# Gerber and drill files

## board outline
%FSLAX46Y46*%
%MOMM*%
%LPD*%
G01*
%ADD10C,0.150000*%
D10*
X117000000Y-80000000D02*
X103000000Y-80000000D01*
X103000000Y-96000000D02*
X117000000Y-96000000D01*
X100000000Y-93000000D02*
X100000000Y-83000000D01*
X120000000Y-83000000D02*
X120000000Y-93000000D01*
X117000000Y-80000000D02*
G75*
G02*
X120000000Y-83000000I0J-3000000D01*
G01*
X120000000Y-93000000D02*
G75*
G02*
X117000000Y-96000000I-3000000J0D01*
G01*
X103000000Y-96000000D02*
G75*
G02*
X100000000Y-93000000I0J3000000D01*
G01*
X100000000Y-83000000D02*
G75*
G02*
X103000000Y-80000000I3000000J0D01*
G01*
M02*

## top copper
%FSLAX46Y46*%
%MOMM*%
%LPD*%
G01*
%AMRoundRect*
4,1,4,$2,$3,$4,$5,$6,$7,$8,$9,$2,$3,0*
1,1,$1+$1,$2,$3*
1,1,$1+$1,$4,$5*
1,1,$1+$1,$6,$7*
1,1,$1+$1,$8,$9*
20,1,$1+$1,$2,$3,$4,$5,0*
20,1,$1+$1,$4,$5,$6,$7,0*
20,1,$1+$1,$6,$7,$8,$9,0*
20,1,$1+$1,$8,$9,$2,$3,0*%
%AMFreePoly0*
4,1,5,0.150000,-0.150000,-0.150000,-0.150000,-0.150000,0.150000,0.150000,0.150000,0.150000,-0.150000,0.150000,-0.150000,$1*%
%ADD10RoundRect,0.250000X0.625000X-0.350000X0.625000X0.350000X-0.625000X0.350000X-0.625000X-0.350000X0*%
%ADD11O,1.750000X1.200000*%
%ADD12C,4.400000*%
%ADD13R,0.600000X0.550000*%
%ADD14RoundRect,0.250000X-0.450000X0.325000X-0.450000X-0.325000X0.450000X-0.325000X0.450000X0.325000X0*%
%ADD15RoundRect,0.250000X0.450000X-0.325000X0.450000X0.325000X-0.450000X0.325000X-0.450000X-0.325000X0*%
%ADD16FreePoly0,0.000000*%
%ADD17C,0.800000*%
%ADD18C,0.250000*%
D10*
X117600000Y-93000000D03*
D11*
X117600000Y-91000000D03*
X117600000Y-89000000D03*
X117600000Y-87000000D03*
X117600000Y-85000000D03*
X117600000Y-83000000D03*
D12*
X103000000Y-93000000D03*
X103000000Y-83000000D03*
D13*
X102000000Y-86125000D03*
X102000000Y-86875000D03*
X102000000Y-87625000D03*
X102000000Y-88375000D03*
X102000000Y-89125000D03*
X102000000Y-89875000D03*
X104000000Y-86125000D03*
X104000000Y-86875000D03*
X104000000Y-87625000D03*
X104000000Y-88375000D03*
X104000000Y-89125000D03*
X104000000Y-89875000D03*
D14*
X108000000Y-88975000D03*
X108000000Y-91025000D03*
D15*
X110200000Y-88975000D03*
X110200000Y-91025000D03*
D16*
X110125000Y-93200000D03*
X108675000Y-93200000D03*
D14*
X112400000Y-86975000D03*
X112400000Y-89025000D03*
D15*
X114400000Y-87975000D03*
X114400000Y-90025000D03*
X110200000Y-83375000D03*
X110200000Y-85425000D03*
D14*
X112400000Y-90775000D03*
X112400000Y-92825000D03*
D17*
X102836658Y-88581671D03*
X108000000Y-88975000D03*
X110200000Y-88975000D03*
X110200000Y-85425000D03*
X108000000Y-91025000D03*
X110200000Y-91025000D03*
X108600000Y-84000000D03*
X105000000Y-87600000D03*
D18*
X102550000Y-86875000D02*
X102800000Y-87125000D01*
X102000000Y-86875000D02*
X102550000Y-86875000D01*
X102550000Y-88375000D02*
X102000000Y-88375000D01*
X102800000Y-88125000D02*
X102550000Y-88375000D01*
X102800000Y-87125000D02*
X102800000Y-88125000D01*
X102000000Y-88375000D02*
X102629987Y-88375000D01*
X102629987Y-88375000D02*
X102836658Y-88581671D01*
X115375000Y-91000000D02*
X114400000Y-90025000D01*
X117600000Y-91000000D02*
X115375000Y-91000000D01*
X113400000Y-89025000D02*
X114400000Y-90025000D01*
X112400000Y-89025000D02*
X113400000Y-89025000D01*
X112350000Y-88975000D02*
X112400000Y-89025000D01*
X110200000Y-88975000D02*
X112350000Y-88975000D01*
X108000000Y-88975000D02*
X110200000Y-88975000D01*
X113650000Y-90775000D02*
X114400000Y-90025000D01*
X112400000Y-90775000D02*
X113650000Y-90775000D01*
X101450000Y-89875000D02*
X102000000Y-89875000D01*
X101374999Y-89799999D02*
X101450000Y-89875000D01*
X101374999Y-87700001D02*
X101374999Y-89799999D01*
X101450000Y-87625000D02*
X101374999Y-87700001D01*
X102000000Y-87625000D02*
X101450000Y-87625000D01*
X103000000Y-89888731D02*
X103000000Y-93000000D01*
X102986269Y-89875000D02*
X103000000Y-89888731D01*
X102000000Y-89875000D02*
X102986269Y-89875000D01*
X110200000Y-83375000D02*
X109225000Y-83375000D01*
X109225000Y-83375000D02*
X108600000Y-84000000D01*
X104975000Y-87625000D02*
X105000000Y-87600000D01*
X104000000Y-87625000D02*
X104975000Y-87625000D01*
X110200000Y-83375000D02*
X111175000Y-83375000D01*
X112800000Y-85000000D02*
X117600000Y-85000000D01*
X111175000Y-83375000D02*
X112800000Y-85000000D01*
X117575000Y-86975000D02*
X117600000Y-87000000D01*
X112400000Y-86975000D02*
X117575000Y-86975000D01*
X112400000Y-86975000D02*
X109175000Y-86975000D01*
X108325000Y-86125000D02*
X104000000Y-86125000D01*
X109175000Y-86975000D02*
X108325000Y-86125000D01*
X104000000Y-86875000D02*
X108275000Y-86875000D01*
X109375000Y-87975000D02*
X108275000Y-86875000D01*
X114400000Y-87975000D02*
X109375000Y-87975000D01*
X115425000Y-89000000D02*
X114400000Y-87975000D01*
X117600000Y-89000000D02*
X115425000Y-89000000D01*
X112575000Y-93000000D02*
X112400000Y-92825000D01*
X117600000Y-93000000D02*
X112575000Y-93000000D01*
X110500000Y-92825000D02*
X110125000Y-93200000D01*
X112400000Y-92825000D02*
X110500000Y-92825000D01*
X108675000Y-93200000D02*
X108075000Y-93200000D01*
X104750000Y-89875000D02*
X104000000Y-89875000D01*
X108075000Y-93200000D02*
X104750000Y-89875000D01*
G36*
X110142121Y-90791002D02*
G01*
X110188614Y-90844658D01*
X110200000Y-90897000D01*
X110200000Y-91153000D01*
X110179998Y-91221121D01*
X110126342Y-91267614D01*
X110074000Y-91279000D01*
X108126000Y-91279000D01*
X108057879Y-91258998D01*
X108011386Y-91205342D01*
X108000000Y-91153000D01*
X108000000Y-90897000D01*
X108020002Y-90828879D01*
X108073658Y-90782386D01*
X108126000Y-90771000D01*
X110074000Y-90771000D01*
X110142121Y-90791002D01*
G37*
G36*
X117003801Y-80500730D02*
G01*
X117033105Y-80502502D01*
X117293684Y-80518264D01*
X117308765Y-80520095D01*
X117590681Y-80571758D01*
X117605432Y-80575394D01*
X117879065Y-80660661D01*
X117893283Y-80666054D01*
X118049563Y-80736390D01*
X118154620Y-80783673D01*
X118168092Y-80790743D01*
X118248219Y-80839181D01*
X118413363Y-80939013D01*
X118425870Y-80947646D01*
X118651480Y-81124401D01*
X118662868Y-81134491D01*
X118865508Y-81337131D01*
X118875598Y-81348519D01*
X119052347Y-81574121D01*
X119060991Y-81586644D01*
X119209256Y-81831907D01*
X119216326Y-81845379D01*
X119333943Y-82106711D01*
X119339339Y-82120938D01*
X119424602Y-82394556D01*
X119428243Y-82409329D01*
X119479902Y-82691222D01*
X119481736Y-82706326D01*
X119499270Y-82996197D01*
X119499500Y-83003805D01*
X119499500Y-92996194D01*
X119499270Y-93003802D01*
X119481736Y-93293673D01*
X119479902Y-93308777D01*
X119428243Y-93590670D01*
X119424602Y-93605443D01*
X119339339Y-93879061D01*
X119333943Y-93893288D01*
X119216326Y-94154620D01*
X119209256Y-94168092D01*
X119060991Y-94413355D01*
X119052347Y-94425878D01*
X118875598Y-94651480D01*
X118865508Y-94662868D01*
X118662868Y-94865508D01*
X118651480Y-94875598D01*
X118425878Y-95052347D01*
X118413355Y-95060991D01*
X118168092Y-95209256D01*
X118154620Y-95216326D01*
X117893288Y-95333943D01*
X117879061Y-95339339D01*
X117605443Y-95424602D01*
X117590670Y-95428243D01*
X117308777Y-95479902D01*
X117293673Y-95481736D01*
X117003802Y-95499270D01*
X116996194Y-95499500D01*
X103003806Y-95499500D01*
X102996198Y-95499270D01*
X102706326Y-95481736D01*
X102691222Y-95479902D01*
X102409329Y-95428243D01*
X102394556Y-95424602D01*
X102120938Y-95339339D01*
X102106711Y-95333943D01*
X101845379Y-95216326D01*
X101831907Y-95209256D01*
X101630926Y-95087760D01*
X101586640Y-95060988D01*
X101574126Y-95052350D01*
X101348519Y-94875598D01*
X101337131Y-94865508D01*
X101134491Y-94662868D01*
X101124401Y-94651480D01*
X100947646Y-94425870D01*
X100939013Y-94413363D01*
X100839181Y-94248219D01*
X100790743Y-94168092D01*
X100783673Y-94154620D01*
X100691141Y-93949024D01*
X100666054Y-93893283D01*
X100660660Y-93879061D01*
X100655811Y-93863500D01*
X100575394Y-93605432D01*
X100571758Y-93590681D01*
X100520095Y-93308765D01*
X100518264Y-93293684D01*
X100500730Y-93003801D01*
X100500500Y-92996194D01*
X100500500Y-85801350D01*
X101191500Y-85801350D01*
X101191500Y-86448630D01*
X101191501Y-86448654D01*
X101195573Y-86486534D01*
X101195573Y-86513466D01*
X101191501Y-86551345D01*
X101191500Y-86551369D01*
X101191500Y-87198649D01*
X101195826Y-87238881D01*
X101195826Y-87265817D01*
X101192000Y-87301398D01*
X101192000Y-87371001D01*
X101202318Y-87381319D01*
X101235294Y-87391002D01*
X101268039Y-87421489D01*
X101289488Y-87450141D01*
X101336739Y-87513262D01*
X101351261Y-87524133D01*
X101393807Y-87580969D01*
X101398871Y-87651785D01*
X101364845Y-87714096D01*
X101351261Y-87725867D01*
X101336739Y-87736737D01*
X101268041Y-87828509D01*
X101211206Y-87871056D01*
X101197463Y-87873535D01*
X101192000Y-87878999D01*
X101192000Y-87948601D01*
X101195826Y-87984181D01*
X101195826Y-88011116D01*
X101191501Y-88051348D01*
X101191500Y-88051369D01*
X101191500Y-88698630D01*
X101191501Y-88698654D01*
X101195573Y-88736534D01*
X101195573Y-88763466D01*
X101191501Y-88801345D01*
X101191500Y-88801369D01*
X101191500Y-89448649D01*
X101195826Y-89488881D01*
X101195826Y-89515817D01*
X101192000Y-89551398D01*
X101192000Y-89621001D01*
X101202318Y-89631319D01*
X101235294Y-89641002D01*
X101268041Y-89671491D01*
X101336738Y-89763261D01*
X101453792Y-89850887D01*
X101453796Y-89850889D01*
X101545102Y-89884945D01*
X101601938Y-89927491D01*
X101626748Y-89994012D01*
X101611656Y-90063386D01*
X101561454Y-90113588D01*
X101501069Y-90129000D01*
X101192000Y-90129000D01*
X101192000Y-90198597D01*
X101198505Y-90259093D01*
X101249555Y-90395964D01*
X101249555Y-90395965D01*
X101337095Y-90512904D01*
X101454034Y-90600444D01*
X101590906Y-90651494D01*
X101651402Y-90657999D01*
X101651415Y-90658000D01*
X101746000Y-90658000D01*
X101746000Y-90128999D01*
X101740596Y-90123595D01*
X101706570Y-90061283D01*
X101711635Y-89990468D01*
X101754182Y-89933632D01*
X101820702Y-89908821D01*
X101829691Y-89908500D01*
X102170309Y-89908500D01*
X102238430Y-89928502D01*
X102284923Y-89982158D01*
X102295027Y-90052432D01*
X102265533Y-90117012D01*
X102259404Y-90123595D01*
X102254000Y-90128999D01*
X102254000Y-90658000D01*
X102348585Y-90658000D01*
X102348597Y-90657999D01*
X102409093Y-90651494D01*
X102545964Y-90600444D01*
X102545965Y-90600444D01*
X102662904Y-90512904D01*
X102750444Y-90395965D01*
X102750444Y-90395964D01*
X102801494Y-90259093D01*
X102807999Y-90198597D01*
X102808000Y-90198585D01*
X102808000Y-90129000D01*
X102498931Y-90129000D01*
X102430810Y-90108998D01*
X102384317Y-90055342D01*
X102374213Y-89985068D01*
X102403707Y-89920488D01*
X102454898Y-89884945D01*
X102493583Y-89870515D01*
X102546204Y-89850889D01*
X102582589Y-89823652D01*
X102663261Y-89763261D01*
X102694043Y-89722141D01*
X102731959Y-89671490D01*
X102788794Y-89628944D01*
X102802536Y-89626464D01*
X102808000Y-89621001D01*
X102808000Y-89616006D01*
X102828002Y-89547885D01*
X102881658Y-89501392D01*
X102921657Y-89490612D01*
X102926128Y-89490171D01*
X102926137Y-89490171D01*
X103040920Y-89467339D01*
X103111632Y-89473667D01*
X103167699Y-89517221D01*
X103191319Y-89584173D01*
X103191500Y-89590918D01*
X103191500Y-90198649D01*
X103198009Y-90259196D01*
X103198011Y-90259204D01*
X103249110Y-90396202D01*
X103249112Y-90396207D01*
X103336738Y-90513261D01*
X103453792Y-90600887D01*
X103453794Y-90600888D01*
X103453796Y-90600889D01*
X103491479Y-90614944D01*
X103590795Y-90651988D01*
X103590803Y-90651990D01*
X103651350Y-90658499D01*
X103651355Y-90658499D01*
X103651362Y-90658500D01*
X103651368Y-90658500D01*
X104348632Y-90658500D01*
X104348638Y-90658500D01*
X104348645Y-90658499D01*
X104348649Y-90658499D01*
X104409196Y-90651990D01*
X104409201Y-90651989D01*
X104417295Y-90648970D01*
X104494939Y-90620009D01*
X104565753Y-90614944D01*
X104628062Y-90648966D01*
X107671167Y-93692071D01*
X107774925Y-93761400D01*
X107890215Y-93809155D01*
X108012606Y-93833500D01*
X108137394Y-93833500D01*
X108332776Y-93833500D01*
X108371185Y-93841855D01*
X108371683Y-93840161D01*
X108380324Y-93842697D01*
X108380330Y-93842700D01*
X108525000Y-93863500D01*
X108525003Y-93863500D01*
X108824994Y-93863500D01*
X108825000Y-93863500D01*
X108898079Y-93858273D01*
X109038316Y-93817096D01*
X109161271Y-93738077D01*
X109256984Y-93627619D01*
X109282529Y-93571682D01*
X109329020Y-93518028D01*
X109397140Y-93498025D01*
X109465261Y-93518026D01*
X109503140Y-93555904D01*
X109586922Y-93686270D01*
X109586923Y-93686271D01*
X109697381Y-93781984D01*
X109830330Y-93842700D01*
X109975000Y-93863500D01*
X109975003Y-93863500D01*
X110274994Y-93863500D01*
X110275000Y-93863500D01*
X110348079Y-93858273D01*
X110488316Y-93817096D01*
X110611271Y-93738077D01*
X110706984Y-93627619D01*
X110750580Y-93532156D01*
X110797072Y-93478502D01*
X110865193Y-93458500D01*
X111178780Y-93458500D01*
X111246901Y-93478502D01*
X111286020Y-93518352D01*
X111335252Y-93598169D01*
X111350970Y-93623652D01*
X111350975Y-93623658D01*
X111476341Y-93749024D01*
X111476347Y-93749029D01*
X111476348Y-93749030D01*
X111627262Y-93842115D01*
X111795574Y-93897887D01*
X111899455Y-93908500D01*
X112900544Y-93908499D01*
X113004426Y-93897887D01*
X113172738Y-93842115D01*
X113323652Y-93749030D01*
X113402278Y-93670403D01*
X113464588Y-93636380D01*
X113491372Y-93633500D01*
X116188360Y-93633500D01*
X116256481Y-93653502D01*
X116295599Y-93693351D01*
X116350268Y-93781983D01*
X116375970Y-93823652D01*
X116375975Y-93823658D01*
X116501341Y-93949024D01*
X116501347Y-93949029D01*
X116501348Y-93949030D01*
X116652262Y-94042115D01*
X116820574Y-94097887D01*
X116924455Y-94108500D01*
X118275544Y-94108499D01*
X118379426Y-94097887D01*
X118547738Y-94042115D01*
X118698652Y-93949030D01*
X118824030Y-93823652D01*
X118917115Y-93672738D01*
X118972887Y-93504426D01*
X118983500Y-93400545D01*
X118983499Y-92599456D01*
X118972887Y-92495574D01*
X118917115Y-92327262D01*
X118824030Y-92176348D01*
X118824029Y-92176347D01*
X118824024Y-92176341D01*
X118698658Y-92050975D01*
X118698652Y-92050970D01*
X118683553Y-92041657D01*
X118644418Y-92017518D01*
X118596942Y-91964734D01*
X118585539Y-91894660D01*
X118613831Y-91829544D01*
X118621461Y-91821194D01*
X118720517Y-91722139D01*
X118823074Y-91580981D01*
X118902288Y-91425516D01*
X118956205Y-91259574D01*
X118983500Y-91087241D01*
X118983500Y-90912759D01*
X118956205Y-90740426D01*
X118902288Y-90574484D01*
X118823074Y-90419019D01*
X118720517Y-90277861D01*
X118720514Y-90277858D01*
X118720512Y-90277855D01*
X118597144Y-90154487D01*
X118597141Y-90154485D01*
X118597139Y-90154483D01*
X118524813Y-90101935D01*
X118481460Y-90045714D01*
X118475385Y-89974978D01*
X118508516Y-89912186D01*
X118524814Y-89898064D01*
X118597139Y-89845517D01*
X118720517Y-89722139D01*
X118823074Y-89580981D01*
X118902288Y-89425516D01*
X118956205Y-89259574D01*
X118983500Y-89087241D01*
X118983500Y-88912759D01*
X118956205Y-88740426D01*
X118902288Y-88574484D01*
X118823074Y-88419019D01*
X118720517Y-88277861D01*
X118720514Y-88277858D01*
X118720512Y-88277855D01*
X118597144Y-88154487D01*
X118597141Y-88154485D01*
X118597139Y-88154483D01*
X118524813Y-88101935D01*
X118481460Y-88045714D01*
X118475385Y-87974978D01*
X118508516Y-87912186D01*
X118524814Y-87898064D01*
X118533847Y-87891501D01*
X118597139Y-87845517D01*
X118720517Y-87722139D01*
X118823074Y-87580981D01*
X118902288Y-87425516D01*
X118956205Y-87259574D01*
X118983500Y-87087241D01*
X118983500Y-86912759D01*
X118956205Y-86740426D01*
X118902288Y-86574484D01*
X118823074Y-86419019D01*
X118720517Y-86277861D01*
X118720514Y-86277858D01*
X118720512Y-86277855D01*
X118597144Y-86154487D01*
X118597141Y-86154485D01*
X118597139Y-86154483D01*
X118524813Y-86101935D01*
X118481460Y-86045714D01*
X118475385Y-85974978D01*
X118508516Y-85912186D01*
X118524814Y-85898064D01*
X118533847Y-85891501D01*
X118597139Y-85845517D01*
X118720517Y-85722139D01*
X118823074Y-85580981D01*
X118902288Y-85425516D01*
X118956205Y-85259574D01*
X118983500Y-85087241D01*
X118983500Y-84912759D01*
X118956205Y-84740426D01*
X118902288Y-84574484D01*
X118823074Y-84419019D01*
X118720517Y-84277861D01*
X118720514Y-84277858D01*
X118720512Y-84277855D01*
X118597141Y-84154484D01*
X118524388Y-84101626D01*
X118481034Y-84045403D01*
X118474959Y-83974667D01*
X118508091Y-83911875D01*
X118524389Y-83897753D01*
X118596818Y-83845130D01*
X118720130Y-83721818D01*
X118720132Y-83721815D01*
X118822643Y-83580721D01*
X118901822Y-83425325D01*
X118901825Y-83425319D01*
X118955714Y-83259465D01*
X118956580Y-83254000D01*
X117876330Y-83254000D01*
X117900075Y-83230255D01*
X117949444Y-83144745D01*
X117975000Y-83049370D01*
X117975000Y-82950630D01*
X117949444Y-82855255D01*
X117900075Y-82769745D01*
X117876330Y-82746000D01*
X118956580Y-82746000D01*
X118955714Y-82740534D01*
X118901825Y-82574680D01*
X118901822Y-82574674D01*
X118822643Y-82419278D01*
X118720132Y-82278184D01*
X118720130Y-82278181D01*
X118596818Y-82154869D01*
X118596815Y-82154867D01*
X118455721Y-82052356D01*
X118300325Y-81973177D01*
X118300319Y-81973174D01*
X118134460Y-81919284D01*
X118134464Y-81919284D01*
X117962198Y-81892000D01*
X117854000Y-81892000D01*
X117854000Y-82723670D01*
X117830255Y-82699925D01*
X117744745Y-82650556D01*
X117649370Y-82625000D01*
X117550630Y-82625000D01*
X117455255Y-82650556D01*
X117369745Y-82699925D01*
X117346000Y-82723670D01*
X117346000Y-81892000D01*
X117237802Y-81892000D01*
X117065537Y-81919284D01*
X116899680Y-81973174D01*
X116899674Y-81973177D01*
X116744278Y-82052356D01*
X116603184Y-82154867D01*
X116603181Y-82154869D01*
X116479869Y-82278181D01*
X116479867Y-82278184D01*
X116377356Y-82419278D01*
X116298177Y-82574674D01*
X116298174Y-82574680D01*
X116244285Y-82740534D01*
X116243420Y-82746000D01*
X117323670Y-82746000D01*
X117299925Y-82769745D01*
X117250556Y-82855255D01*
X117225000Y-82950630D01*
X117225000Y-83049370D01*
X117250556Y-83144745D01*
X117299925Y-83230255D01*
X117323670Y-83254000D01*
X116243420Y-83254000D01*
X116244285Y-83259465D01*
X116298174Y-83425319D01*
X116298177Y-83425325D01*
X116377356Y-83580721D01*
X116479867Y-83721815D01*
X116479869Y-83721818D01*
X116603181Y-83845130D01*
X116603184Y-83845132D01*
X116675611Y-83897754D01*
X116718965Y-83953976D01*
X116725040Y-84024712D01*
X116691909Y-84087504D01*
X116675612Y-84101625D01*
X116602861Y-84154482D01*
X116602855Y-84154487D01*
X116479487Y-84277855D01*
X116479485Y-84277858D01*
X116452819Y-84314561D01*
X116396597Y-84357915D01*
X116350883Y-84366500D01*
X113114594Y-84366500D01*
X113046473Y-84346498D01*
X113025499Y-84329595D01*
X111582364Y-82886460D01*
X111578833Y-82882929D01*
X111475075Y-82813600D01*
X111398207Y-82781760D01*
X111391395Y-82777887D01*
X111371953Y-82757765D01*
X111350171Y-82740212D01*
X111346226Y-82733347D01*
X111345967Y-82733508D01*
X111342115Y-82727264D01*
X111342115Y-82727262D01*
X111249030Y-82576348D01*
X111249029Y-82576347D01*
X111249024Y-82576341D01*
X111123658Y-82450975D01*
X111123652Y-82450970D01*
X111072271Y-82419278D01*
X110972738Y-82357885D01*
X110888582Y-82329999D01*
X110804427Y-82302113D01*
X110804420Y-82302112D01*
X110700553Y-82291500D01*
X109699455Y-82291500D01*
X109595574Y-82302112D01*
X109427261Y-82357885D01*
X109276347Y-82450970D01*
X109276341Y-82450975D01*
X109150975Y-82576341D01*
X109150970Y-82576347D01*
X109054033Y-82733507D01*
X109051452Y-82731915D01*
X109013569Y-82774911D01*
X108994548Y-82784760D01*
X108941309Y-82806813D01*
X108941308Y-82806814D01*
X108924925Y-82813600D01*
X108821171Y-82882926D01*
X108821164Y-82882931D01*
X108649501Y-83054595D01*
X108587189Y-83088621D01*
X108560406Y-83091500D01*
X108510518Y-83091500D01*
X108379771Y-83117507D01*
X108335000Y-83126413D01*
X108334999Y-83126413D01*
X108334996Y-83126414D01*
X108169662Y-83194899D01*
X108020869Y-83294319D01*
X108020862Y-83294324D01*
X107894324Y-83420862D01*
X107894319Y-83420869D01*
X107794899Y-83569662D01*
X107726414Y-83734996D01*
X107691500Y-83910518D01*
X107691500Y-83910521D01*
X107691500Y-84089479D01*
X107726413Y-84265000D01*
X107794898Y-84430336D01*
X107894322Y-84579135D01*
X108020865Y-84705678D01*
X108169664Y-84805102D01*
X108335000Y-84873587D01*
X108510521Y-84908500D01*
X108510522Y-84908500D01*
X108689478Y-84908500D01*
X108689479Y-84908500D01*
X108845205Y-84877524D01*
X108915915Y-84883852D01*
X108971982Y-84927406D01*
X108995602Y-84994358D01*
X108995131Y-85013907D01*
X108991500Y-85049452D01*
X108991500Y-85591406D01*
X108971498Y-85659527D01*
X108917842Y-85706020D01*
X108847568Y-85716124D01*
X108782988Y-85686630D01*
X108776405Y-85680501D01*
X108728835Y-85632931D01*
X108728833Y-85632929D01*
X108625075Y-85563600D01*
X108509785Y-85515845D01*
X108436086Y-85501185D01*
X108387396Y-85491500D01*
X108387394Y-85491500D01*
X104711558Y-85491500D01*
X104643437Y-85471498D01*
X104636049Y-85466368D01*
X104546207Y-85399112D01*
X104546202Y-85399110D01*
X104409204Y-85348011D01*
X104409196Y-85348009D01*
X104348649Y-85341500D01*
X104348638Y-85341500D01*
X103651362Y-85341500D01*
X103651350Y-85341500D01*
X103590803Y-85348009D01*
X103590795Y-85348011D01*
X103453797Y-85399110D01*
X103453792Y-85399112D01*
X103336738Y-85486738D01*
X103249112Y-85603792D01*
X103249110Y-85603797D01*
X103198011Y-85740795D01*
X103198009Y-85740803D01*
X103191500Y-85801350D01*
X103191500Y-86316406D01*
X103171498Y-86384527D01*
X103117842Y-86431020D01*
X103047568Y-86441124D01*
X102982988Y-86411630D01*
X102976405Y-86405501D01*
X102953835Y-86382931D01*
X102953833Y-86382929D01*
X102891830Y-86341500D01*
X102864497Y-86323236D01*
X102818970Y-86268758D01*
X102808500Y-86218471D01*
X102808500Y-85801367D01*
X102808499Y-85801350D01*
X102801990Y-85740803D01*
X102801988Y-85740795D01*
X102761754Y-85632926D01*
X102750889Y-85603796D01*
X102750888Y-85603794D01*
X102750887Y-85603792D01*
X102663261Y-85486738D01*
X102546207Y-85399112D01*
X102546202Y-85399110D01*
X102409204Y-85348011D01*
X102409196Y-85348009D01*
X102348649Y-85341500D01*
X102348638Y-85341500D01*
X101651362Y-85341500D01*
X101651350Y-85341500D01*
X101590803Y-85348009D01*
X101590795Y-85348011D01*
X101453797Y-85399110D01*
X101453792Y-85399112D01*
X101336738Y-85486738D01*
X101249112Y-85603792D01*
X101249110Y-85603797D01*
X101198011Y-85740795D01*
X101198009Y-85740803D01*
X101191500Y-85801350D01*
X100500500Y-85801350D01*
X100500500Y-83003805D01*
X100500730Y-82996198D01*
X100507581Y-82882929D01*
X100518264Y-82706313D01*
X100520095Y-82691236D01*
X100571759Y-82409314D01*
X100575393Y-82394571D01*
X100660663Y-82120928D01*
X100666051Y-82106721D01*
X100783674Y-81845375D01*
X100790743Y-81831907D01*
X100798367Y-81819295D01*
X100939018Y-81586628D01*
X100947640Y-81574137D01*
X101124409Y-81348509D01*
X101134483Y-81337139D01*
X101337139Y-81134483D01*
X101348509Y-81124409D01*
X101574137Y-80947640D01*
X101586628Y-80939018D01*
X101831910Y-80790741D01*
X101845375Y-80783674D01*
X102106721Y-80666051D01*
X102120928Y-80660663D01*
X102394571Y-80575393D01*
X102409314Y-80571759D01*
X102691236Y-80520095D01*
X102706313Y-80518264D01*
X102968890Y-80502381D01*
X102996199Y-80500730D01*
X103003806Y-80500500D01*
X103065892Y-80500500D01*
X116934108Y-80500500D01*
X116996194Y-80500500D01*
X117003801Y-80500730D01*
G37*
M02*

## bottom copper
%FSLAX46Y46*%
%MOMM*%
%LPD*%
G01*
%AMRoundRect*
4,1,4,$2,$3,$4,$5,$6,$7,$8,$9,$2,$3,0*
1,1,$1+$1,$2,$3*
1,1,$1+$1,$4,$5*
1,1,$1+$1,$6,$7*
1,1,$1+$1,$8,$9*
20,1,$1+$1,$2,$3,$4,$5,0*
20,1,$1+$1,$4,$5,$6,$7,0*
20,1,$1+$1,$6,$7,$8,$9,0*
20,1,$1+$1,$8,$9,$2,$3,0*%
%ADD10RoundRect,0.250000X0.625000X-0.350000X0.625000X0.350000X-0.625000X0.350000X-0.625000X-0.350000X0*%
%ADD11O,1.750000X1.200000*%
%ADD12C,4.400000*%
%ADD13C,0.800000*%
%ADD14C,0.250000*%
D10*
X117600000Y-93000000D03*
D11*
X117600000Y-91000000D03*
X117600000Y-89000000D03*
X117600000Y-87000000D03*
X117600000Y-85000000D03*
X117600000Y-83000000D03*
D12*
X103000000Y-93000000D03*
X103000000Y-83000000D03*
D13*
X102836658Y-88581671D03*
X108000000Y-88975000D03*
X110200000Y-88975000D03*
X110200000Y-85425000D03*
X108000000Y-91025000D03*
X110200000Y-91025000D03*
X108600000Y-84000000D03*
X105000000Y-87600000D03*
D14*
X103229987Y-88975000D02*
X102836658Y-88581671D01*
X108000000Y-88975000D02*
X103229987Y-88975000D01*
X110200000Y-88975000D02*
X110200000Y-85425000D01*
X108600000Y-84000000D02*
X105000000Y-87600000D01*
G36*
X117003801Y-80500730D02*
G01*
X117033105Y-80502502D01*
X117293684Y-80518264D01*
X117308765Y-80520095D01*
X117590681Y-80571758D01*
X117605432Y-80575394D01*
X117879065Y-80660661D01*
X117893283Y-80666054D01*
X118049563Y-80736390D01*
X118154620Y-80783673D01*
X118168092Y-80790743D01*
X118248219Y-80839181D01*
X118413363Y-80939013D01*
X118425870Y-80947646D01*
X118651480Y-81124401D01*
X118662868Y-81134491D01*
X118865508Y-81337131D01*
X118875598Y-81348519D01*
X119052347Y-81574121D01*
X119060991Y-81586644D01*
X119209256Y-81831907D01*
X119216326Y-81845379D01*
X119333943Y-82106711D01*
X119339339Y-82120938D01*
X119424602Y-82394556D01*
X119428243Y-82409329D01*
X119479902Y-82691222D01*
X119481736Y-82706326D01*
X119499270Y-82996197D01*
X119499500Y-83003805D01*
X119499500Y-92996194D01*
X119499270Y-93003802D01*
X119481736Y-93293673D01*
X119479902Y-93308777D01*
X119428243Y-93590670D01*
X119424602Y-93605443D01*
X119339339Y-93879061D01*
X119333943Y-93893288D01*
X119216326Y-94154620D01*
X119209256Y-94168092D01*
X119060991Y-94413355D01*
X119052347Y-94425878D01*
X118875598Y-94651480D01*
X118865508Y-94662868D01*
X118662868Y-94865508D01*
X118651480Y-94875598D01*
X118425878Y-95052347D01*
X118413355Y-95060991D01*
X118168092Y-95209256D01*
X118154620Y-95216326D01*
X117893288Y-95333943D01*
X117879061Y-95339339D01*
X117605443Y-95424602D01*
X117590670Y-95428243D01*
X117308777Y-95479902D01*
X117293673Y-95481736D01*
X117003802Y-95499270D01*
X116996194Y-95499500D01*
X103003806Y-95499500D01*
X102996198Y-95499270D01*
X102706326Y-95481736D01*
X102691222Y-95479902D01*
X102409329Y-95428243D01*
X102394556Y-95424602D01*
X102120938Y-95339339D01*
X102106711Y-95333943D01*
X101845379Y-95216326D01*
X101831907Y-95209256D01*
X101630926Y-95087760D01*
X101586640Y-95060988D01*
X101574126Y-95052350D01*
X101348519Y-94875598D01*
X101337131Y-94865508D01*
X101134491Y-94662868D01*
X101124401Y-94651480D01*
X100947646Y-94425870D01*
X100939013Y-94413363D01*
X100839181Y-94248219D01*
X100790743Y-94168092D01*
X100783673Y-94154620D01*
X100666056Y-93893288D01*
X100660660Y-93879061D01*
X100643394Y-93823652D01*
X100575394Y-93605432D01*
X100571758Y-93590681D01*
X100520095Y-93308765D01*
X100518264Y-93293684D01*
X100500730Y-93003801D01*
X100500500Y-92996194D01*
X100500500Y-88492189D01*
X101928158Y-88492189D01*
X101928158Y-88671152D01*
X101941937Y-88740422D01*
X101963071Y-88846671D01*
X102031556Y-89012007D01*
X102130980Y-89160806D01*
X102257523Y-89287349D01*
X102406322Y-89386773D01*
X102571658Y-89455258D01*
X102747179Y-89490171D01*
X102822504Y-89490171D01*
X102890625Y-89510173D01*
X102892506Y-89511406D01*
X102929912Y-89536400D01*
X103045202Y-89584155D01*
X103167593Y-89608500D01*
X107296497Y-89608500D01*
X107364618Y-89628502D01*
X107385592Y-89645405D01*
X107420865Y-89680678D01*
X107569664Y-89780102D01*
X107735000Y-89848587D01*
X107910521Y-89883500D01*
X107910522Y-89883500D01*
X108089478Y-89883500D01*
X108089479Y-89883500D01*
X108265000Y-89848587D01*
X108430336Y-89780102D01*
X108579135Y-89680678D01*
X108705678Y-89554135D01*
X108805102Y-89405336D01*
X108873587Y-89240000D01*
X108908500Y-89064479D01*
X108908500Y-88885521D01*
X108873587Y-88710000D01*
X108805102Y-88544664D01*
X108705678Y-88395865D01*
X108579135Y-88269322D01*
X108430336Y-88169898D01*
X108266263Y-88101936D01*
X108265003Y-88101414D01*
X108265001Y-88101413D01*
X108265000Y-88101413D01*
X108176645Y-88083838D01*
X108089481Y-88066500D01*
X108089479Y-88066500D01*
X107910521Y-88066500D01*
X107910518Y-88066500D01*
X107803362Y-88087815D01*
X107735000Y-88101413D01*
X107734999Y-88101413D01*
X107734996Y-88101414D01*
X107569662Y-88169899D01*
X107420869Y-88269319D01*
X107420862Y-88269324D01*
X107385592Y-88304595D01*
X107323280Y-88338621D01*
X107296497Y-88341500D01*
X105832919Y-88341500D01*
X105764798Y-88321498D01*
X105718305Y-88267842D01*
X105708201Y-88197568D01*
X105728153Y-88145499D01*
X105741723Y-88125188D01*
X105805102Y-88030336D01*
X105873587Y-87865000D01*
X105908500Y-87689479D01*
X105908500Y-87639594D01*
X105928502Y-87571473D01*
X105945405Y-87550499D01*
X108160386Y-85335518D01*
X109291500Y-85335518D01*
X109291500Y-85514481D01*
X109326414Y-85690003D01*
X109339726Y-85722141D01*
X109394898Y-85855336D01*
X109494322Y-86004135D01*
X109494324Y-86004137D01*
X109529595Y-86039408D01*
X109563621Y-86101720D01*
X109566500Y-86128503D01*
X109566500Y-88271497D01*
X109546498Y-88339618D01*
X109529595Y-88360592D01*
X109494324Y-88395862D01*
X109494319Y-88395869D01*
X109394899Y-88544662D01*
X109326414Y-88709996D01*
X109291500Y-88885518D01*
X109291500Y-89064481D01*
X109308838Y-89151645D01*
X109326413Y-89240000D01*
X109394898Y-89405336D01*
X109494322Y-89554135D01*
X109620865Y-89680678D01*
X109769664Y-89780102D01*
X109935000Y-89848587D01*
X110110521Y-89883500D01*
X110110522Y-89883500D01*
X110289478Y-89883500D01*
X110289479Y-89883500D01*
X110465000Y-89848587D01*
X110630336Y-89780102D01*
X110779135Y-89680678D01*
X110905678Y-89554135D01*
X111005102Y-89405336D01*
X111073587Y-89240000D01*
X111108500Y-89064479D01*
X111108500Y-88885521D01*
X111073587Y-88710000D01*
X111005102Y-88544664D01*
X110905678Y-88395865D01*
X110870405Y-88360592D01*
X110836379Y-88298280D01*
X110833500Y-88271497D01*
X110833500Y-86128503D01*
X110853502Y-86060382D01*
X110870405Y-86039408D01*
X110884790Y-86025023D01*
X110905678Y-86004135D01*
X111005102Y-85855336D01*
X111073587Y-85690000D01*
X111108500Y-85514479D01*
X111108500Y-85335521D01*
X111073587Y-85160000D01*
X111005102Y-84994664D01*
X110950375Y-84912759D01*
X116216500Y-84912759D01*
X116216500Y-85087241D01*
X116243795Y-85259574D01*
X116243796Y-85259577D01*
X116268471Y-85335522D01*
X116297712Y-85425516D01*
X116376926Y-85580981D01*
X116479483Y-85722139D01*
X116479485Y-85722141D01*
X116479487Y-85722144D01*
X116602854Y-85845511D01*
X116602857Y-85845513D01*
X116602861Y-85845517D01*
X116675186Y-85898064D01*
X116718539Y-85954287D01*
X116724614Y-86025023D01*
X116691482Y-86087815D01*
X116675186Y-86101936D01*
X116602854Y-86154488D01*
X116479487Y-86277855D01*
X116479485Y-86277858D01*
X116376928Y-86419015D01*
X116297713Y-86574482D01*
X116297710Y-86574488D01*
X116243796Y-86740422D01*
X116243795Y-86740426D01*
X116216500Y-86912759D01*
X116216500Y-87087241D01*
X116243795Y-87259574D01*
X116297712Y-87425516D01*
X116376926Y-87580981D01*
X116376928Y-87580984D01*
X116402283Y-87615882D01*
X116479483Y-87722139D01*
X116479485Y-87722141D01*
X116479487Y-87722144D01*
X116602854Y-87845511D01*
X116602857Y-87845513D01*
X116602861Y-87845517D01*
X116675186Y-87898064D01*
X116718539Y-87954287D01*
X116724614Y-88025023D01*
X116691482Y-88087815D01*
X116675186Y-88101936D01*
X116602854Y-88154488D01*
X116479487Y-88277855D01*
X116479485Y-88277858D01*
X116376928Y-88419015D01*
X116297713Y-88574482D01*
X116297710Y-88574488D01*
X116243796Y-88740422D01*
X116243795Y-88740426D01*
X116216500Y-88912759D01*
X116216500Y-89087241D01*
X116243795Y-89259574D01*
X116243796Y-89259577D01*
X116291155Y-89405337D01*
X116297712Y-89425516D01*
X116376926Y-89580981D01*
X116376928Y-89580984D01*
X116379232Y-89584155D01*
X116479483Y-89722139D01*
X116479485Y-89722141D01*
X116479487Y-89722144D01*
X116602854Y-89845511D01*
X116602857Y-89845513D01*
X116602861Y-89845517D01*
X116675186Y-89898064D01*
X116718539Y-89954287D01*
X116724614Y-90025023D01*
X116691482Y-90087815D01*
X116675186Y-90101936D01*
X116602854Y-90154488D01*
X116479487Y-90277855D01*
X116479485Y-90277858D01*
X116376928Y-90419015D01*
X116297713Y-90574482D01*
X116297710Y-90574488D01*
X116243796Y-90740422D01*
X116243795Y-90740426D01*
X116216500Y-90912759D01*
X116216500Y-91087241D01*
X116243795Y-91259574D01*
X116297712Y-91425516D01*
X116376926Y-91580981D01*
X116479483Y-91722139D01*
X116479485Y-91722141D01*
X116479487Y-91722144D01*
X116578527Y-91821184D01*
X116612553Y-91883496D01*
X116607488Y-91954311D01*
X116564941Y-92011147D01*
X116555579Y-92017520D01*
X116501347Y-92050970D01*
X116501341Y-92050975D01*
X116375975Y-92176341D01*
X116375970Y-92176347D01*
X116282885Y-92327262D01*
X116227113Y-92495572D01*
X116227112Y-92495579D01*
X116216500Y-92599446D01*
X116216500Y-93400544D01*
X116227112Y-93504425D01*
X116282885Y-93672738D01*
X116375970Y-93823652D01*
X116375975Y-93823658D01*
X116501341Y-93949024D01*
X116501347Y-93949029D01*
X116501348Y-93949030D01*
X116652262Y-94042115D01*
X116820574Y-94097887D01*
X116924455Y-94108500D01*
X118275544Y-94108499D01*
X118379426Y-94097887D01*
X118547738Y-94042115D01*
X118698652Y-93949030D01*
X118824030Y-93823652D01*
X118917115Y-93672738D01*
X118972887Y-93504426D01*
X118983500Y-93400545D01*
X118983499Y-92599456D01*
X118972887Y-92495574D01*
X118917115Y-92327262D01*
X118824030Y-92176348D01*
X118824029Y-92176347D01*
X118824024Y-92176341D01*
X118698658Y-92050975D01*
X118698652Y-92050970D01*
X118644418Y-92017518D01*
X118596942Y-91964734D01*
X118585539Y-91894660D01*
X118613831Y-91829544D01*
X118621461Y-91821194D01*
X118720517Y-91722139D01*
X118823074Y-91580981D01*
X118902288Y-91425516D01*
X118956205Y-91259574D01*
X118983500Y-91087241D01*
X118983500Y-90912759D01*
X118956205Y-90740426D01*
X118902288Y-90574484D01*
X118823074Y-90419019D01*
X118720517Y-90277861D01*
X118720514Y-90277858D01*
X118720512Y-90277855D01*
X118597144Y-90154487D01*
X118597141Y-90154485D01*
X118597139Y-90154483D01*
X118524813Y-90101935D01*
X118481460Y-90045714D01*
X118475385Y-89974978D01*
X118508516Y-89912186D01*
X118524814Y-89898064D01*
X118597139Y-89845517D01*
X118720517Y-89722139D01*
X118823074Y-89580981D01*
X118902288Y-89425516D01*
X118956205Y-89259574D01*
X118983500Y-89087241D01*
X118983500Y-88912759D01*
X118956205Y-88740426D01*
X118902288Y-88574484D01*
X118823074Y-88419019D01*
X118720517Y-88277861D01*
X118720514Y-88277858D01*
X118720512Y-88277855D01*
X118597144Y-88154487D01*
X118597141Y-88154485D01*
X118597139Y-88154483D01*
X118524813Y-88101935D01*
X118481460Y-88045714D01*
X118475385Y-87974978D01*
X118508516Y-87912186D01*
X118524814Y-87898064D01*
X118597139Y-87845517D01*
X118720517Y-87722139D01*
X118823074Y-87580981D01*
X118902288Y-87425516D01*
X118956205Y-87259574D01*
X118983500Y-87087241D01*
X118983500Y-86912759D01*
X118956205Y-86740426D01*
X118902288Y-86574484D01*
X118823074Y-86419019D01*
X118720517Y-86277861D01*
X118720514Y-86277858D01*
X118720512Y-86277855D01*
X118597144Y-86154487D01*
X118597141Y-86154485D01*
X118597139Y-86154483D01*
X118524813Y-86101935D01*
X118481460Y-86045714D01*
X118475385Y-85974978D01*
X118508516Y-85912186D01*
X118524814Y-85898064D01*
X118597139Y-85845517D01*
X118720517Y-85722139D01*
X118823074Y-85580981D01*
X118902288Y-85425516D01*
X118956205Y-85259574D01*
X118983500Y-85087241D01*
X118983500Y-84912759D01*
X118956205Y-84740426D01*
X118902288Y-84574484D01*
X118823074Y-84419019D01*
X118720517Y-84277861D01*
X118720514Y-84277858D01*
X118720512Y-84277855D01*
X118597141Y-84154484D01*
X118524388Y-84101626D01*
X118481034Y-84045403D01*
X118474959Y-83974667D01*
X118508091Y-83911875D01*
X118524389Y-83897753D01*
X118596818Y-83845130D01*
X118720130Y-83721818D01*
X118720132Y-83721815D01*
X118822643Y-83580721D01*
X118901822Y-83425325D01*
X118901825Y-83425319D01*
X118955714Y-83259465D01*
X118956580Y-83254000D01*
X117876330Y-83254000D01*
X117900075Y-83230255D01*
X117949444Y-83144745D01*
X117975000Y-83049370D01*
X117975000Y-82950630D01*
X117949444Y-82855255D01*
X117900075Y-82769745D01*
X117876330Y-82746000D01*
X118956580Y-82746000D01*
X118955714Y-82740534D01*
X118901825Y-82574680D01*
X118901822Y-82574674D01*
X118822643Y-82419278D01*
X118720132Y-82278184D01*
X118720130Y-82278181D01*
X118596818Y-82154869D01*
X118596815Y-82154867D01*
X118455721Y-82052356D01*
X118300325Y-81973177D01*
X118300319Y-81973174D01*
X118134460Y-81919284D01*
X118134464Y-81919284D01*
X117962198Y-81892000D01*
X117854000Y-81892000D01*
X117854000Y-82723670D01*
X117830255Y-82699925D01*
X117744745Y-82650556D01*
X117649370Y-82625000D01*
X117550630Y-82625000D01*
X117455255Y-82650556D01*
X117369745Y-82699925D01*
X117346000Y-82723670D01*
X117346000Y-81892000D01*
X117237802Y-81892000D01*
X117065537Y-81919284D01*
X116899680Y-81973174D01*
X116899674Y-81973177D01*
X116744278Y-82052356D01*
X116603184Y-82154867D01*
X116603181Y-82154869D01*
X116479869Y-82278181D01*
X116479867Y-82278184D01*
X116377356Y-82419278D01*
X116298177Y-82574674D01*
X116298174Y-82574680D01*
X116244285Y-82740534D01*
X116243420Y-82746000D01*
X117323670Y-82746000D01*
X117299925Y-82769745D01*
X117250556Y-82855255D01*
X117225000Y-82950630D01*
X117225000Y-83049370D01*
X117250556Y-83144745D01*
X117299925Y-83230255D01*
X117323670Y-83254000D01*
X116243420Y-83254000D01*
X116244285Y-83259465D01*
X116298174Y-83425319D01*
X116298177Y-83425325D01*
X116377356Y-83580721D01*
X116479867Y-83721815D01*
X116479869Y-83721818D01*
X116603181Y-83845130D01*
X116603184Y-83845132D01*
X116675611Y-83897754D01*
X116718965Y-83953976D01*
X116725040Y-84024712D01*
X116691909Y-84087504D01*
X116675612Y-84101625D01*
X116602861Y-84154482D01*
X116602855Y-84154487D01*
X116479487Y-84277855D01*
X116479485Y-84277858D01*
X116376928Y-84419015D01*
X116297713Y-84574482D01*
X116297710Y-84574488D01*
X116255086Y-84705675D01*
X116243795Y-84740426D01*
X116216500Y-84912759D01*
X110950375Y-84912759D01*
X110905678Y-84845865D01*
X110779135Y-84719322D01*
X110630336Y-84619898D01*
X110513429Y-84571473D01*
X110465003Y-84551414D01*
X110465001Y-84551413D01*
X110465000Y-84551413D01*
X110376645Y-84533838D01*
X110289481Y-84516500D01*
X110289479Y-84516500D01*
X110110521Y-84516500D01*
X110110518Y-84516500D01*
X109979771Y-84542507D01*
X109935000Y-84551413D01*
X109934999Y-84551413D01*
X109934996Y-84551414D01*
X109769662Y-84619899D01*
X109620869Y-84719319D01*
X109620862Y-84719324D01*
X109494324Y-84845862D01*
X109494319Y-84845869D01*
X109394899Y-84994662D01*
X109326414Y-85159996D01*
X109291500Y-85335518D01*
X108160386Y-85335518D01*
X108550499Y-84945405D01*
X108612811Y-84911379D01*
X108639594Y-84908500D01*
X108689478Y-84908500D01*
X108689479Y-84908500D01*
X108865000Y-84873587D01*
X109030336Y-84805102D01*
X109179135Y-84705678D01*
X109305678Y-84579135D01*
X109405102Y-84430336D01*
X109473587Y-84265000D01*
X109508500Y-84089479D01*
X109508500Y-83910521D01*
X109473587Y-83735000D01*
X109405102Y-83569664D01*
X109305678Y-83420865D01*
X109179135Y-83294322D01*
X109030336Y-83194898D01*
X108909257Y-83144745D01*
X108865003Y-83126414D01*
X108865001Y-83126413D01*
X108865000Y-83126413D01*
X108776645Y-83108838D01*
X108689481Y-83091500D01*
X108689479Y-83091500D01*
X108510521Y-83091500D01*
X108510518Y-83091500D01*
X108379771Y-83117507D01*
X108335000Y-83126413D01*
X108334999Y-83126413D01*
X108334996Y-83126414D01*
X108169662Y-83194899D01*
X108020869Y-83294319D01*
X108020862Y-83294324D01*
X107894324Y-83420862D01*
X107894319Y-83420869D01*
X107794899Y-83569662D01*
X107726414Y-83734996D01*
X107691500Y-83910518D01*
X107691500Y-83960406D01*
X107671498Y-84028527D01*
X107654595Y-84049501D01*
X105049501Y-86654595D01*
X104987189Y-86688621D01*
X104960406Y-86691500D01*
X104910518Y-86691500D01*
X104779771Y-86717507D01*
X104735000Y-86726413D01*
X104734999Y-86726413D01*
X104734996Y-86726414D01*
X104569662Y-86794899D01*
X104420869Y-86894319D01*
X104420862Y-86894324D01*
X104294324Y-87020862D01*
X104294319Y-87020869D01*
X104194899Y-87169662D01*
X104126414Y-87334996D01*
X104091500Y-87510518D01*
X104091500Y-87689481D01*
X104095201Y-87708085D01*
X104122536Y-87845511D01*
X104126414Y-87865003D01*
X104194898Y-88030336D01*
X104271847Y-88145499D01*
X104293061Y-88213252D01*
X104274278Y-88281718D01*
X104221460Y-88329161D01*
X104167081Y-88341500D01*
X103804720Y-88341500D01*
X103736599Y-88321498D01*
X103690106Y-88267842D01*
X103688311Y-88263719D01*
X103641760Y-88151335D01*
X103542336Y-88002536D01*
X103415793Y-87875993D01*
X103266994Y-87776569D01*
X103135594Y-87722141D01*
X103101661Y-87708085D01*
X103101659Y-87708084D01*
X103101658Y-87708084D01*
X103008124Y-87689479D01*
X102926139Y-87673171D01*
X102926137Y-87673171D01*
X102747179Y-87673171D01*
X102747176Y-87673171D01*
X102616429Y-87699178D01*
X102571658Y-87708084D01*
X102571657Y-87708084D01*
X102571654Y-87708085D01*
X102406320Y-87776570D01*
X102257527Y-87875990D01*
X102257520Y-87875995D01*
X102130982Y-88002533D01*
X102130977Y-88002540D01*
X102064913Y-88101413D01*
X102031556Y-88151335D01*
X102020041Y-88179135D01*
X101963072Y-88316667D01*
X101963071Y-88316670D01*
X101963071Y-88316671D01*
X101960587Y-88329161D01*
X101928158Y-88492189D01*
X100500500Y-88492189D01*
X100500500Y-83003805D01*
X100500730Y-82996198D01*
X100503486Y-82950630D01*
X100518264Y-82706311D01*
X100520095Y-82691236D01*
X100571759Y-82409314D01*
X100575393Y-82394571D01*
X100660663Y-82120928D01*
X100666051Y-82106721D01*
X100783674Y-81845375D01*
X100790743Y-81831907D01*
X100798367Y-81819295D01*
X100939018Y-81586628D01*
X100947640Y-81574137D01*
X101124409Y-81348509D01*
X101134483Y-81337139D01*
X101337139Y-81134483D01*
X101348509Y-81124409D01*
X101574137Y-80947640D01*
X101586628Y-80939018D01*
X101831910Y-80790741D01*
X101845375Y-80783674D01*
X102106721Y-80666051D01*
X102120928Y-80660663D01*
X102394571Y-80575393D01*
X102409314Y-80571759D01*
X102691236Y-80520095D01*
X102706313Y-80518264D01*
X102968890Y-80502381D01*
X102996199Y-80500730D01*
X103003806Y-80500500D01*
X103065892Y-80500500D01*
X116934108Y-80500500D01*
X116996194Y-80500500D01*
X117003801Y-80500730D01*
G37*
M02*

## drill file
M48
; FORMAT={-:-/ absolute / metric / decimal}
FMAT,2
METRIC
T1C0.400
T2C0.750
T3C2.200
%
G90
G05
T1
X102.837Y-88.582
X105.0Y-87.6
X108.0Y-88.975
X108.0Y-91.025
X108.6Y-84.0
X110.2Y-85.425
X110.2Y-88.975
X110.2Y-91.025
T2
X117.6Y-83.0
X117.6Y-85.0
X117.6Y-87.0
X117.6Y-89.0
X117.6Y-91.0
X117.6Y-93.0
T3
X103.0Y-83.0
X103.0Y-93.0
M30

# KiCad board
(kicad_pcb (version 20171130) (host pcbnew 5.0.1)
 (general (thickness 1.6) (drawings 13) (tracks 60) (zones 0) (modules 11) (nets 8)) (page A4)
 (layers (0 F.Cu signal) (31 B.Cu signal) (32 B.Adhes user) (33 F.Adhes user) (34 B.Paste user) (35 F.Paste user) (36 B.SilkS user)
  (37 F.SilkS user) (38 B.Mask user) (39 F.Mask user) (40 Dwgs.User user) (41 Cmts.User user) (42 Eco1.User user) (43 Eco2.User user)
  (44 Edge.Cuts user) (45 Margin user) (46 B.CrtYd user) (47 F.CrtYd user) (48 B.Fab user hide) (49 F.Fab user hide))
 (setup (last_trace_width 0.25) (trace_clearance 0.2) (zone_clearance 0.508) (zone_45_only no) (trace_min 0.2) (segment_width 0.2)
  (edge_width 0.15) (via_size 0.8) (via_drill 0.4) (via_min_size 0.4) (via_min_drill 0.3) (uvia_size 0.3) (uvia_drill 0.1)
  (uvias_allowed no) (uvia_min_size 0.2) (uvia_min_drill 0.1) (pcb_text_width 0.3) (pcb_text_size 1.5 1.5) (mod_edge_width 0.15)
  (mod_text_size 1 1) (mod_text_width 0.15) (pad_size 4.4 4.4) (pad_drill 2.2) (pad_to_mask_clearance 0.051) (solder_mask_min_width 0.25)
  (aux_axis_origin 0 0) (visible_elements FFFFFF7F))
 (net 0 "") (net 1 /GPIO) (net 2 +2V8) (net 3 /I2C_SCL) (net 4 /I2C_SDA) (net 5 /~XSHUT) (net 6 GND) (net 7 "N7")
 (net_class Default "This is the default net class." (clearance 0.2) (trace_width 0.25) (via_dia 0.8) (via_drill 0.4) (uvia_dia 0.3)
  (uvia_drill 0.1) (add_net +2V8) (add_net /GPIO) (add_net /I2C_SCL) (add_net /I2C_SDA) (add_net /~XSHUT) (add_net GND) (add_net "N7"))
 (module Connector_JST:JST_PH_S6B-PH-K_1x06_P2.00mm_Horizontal (layer B.Cu) (at 117.6 93 90)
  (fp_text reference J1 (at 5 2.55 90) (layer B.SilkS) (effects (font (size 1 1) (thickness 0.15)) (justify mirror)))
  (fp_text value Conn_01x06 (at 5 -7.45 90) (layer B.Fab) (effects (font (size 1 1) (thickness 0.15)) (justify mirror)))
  (pad 1 thru_hole roundrect (at 0 0 90) (size 1.2 1.75) (drill 0.75) (layers *.Cu *.Mask) (roundrect_rratio 0.208333) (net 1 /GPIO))
  (pad 2 thru_hole oval (at 2 0 90) (size 1.2 1.75) (drill 0.75) (layers *.Cu *.Mask) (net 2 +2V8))
  (pad 3 thru_hole oval (at 4 0 90) (size 1.2 1.75) (drill 0.75) (layers *.Cu *.Mask) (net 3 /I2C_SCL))
  (pad 4 thru_hole oval (at 6 0 90) (size 1.2 1.75) (drill 0.75) (layers *.Cu *.Mask) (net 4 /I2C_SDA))
  (pad 5 thru_hole oval (at 8 0 90) (size 1.2 1.75) (drill 0.75) (layers *.Cu *.Mask) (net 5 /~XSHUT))
  (pad 6 thru_hole oval (at 10 0 90) (size 1.2 1.75) (drill 0.75) (layers *.Cu *.Mask) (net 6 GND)))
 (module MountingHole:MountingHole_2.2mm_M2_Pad (layer F.Cu) (at 103 93)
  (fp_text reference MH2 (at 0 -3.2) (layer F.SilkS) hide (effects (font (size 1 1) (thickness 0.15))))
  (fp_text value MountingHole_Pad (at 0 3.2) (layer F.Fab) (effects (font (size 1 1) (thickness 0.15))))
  (pad 1 thru_hole circle (at 0 0) (size 4.4 4.4) (drill 2.2) (layers *.Cu *.Mask) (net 6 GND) (zone_connect 2)))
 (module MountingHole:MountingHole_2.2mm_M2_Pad (layer F.Cu) (at 103 83)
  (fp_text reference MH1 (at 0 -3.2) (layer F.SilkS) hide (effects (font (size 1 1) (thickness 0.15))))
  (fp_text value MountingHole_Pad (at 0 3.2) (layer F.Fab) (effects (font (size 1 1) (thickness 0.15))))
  (pad 1 thru_hole circle (at 0 0) (size 4.4 4.4) (drill 2.2) (layers *.Cu *.Mask) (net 6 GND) (zone_connect 2)))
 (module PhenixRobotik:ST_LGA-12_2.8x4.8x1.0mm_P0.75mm (layer F.Cu) (at 103 88 180)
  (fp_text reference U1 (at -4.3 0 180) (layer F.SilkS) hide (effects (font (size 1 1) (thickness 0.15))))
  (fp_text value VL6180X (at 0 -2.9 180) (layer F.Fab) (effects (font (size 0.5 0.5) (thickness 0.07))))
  (pad 7 smd rect (at 1 1.875) (size 0.6 0.55) (layers F.Cu F.Paste F.Mask))
  (pad 8 smd rect (at 1 1.125) (size 0.6 0.55) (layers F.Cu F.Paste F.Mask) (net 2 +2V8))
  (pad 9 smd rect (at 1 0.375) (size 0.6 0.55) (layers F.Cu F.Paste F.Mask) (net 6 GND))
  (pad 10 smd rect (at 1 -0.375) (size 0.6 0.55) (layers F.Cu F.Paste F.Mask) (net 2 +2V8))
  (pad 11 smd rect (at 1 -1.125) (size 0.6 0.55) (layers F.Cu F.Paste F.Mask))
  (pad 12 smd rect (at 1 -1.875) (size 0.6 0.55) (layers F.Cu F.Paste F.Mask) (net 6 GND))
  (pad 6 smd rect (at -1 1.875) (size 0.6 0.55) (layers F.Cu F.Paste F.Mask) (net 4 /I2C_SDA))
  (pad 5 smd rect (at -1 1.125) (size 0.6 0.55) (layers F.Cu F.Paste F.Mask) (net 3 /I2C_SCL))
  (pad 4 smd rect (at -1 0.375) (size 0.6 0.55) (layers F.Cu F.Paste F.Mask) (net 5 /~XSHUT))
  (pad 3 smd rect (at -1 -0.375) (size 0.6 0.55) (layers F.Cu F.Paste F.Mask))
  (pad 2 smd rect (at -1 -1.125) (size 0.6 0.55) (layers F.Cu F.Paste F.Mask))
  (pad 1 smd rect (at -1 -1.875) (size 0.6 0.55) (layers F.Cu F.Paste F.Mask) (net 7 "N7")))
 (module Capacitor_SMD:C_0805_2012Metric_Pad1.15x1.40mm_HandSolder (layer F.Cu) (at 108 90 270)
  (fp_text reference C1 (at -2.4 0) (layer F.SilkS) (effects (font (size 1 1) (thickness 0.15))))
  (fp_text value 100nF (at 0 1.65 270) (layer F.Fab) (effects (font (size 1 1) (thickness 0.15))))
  (pad 1 smd roundrect (at -1.025 0 270) (size 1.15 1.4) (layers F.Cu F.Paste F.Mask) (roundrect_rratio 0.217391) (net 2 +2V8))
  (pad 2 smd roundrect (at 1.025 0 270) (size 1.15 1.4) (layers F.Cu F.Paste F.Mask) (roundrect_rratio 0.217391) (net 6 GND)))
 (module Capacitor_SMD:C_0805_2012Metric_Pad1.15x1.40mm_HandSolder (layer F.Cu) (at 110.2 90 90)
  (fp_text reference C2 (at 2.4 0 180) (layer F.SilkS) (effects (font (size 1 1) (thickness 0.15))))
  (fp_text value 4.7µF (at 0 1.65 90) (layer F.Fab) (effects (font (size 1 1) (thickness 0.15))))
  (pad 2 smd roundrect (at 1.025 0 90) (size 1.15 1.4) (layers F.Cu F.Paste F.Mask) (roundrect_rratio 0.217391) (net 2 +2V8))
  (pad 1 smd roundrect (at -1.025 0 90) (size 1.15 1.4) (layers F.Cu F.Paste F.Mask) (roundrect_rratio 0.217391) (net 6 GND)))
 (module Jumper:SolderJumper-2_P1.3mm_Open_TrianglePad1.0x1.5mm (layer F.Cu) (at 109.4 93.2)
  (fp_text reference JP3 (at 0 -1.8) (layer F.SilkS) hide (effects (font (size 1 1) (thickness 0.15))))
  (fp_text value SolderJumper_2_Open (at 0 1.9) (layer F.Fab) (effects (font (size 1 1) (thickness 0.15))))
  (pad 2 smd custom (at 0.725 0) (size 0.3 0.3) (layers F.Cu F.Mask) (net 1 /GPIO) (zone_connect 0)
   (options (clearance outline) (anchor rect)) (primitives))
  (pad 1 smd custom (at -0.725 0) (size 0.3 0.3) (layers F.Cu F.Mask) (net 7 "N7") (zone_connect 0)
   (options (clearance outline) (anchor rect)) (primitives)))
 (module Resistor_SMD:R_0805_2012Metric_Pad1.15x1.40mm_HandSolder (layer F.Cu) (at 112.4 88 270)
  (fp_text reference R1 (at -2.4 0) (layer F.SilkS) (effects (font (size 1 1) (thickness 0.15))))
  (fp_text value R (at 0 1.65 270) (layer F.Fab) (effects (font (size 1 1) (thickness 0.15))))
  (pad 1 smd roundrect (at -1.025 0 270) (size 1.15 1.4) (layers F.Cu F.Paste F.Mask) (roundrect_rratio 0.217391) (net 4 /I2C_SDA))
  (pad 2 smd roundrect (at 1.025 0 270) (size 1.15 1.4) (layers F.Cu F.Paste F.Mask) (roundrect_rratio 0.217391) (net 2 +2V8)))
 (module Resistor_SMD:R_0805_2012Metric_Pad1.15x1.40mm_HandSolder (layer F.Cu) (at 114.4 89 90)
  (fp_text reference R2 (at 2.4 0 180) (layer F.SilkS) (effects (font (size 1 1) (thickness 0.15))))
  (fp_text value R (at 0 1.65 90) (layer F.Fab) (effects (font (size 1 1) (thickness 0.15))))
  (pad 2 smd roundrect (at 1.025 0 90) (size 1.15 1.4) (layers F.Cu F.Paste F.Mask) (roundrect_rratio 0.217391) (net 3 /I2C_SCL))
  (pad 1 smd roundrect (at -1.025 0 90) (size 1.15 1.4) (layers F.Cu F.Paste F.Mask) (roundrect_rratio 0.217391) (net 2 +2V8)))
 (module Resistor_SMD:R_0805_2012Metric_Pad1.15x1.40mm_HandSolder (layer F.Cu) (at 110.2 84.4 90)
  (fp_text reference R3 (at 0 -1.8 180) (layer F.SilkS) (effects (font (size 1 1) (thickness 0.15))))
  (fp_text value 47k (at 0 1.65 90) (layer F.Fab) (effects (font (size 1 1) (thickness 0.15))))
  (pad 2 smd roundrect (at 1.025 0 90) (size 1.15 1.4) (layers F.Cu F.Paste F.Mask) (roundrect_rratio 0.217391) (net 5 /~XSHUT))
  (pad 1 smd roundrect (at -1.025 0 90) (size 1.15 1.4) (layers F.Cu F.Paste F.Mask) (roundrect_rratio 0.217391) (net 2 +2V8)))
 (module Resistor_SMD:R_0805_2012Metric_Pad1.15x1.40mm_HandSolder (layer F.Cu) (at 112.4 91.8 270)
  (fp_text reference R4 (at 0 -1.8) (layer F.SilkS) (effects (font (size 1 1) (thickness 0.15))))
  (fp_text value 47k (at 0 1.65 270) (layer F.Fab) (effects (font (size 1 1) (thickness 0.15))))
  (pad 1 smd roundrect (at -1.025 0 270) (size 1.15 1.4) (layers F.Cu F.Paste F.Mask) (roundrect_rratio 0.217391) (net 2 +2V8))
  (pad 2 smd roundrect (at 1.025 0 270) (size 1.15 1.4) (layers F.Cu F.Paste F.Mask) (roundrect_rratio 0.217391) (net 1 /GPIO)))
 (gr_line (start 117 80) (end 103 80) (layer Edge.Cuts) (width 0.15))
 (gr_line (start 103 96) (end 117 96) (layer Edge.Cuts) (width 0.15))
 (gr_line (start 100 93) (end 100 83) (angle 90) (layer Edge.Cuts) (width 0.15))
 (gr_line (start 120 83) (end 120 93) (angle 90) (layer Edge.Cuts) (width 0.15))
 (gr_arc (start 117 83) (end 117 80) (angle 90) (layer Edge.Cuts) (width 0.15))
 (gr_arc (start 117 93) (end 120 93) (angle 90) (layer Edge.Cuts) (width 0.15))
 (gr_arc (start 103 93) (end 103 96) (angle 90) (layer Edge.Cuts) (width 0.15))
 (gr_arc (start 103 83) (end 100 83) (angle 90) (layer Edge.Cuts) (width 0.15))
 (segment (start 102.55 86.875) (end 102.8 87.125) (width 0.25) (layer F.Cu) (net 2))
 (segment (start 102 86.875) (end 102.55 86.875) (width 0.25) (layer F.Cu) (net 2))
 (segment (start 102.55 88.375) (end 102 88.375) (width 0.25) (layer F.Cu) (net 2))
 (segment (start 102.8 88.125) (end 102.55 88.375) (width 0.25) (layer F.Cu) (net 2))
 (segment (start 102.8 87.125) (end 102.8 88.125) (width 0.25) (layer F.Cu) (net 2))
 (via (at 102.836658 88.581671) (size 0.8) (drill 0.4) (layers F.Cu B.Cu) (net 2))
 (segment (start 102 88.375) (end 102.629987 88.375) (width 0.25) (layer F.Cu) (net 2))
 (segment (start 102.629987 88.375) (end 102.836658 88.581671) (width 0.25) (layer F.Cu) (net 2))
 (segment (start 115.375 91) (end 114.4 90.025) (width 0.25) (layer F.Cu) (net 2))
 (segment (start 117.6 91) (end 115.375 91) (width 0.25) (layer F.Cu) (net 2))
 (segment (start 113.4 89.025) (end 114.4 90.025) (width 0.25) (layer F.Cu) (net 2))
 (segment (start 112.4 89.025) (end 113.4 89.025) (width 0.25) (layer F.Cu) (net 2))
 (segment (start 112.35 88.975) (end 112.4 89.025) (width 0.25) (layer F.Cu) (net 2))
 (segment (start 110.2 88.975) (end 112.35 88.975) (width 0.25) (layer F.Cu) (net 2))
 (segment (start 108 88.975) (end 110.2 88.975) (width 0.25) (layer F.Cu) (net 2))
 (via (at 108 88.975) (size 0.8) (drill 0.4) (layers F.Cu B.Cu) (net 2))
 (segment (start 113.65 90.775) (end 114.4 90.025) (width 0.25) (layer F.Cu) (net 2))
 (segment (start 112.4 90.775) (end 113.65 90.775) (width 0.25) (layer F.Cu) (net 2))
 (segment (start 103.229987 88.975) (end 102.836658 88.581671) (width 0.25) (layer B.Cu) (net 2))
 (segment (start 108 88.975) (end 103.229987 88.975) (width 0.25) (layer B.Cu) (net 2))
 (via (at 110.2 88.975) (size 0.8) (drill 0.4) (layers F.Cu B.Cu) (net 2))
 (via (at 110.2 85.425) (size 0.8) (drill 0.4) (layers F.Cu B.Cu) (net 2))
 (segment (start 110.2 88.975) (end 110.2 85.425) (width 0.25) (layer B.Cu) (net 2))
 (segment (start 101.45 89.875) (end 102 89.875) (width 0.25) (layer F.Cu) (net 6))
 (segment (start 101.374999 89.799999) (end 101.45 89.875) (width 0.25) (layer F.Cu) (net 6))
 (segment (start 101.374999 87.700001) (end 101.374999 89.799999) (width 0.25) (layer F.Cu) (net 6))
 (segment (start 101.45 87.625) (end 101.374999 87.700001) (width 0.25) (layer F.Cu) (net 6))
 (segment (start 102 87.625) (end 101.45 87.625) (width 0.25) (layer F.Cu) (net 6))
 (segment (start 103 89.888731) (end 103 93) (width 0.25) (layer F.Cu) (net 6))
 (segment (start 102.986269 89.875) (end 103 89.888731) (width 0.25) (layer F.Cu) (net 6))
 (segment (start 102 89.875) (end 102.986269 89.875) (width 0.25) (layer F.Cu) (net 6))
 (via (at 108 91.025) (size 0.8) (drill 0.4) (layers F.Cu B.Cu) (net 6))
 (via (at 110.2 91.025) (size 0.8) (drill 0.4) (layers F.Cu B.Cu) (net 6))
 (via (at 108.6 84) (size 0.8) (drill 0.4) (layers F.Cu B.Cu) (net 5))
 (segment (start 110.2 83.375) (end 109.225 83.375) (width 0.25) (layer F.Cu) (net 5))
 (segment (start 109.225 83.375) (end 108.6 84) (width 0.25) (layer F.Cu) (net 5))
 (via (at 105 87.6) (size 0.8) (drill 0.4) (layers F.Cu B.Cu) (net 5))
 (segment (start 108.6 84) (end 105 87.6) (width 0.25) (layer B.Cu) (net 5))
 (segment (start 104.975 87.625) (end 105 87.6) (width 0.25) (layer F.Cu) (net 5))
 (segment (start 104 87.625) (end 104.975 87.625) (width 0.25) (layer F.Cu) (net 5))
 (segment (start 110.2 83.375) (end 111.175 83.375) (width 0.25) (layer F.Cu) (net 5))
 (segment (start 112.8 85) (end 117.6 85) (width 0.25) (layer F.Cu) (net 5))
 (segment (start 111.175 83.375) (end 112.8 85) (width 0.25) (layer F.Cu) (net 5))
 (segment (start 117.575 86.975) (end 117.6 87) (width 0.25) (layer F.Cu) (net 4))
 (segment (start 112.4 86.975) (end 117.575 86.975) (width 0.25) (layer F.Cu) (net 4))
 (segment (start 112.4 86.975) (end 109.175 86.975) (width 0.25) (layer F.Cu) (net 4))
 (segment (start 108.325 86.125) (end 104 86.125) (width 0.25) (layer F.Cu) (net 4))
 (segment (start 109.175 86.975) (end 108.325 86.125) (width 0.25) (layer F.Cu) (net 4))
 (segment (start 104 86.875) (end 108.275 86.875) (width 0.25) (layer F.Cu) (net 3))
 (segment (start 109.375 87.975) (end 108.275 86.875) (width 0.25) (layer F.Cu) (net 3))
 (segment (start 114.4 87.975) (end 109.375 87.975) (width 0.25) (layer F.Cu) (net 3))
 (segment (start 115.425 89) (end 114.4 87.975) (width 0.25) (layer F.Cu) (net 3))
 (segment (start 117.6 89) (end 115.425 89) (width 0.25) (layer F.Cu) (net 3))
 (segment (start 112.575 93) (end 112.4 92.825) (width 0.25) (layer F.Cu) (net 1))
 (segment (start 117.6 93) (end 112.575 93) (width 0.25) (layer F.Cu) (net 1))
 (segment (start 110.5 92.825) (end 110.125 93.2) (width 0.25) (layer F.Cu) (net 1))
 (segment (start 112.4 92.825) (end 110.5 92.825) (width 0.25) (layer F.Cu) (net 1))
 (segment (start 108.675 93.2) (end 108.075 93.2) (width 0.25) (layer F.Cu) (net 7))
 (segment (start 104.75 89.875) (end 104 89.875) (width 0.25) (layer F.Cu) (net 7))
 (segment (start 108.075 93.2) (end 104.75 89.875) (width 0.25) (layer F.Cu) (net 7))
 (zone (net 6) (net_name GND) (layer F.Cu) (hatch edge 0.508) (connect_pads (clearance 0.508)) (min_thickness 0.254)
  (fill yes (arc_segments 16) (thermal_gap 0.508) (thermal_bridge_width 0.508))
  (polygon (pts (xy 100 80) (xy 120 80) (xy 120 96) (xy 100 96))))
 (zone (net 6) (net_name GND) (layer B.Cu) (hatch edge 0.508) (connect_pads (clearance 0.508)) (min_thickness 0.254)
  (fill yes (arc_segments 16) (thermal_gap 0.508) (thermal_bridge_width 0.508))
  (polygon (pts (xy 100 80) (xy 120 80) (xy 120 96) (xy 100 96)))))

